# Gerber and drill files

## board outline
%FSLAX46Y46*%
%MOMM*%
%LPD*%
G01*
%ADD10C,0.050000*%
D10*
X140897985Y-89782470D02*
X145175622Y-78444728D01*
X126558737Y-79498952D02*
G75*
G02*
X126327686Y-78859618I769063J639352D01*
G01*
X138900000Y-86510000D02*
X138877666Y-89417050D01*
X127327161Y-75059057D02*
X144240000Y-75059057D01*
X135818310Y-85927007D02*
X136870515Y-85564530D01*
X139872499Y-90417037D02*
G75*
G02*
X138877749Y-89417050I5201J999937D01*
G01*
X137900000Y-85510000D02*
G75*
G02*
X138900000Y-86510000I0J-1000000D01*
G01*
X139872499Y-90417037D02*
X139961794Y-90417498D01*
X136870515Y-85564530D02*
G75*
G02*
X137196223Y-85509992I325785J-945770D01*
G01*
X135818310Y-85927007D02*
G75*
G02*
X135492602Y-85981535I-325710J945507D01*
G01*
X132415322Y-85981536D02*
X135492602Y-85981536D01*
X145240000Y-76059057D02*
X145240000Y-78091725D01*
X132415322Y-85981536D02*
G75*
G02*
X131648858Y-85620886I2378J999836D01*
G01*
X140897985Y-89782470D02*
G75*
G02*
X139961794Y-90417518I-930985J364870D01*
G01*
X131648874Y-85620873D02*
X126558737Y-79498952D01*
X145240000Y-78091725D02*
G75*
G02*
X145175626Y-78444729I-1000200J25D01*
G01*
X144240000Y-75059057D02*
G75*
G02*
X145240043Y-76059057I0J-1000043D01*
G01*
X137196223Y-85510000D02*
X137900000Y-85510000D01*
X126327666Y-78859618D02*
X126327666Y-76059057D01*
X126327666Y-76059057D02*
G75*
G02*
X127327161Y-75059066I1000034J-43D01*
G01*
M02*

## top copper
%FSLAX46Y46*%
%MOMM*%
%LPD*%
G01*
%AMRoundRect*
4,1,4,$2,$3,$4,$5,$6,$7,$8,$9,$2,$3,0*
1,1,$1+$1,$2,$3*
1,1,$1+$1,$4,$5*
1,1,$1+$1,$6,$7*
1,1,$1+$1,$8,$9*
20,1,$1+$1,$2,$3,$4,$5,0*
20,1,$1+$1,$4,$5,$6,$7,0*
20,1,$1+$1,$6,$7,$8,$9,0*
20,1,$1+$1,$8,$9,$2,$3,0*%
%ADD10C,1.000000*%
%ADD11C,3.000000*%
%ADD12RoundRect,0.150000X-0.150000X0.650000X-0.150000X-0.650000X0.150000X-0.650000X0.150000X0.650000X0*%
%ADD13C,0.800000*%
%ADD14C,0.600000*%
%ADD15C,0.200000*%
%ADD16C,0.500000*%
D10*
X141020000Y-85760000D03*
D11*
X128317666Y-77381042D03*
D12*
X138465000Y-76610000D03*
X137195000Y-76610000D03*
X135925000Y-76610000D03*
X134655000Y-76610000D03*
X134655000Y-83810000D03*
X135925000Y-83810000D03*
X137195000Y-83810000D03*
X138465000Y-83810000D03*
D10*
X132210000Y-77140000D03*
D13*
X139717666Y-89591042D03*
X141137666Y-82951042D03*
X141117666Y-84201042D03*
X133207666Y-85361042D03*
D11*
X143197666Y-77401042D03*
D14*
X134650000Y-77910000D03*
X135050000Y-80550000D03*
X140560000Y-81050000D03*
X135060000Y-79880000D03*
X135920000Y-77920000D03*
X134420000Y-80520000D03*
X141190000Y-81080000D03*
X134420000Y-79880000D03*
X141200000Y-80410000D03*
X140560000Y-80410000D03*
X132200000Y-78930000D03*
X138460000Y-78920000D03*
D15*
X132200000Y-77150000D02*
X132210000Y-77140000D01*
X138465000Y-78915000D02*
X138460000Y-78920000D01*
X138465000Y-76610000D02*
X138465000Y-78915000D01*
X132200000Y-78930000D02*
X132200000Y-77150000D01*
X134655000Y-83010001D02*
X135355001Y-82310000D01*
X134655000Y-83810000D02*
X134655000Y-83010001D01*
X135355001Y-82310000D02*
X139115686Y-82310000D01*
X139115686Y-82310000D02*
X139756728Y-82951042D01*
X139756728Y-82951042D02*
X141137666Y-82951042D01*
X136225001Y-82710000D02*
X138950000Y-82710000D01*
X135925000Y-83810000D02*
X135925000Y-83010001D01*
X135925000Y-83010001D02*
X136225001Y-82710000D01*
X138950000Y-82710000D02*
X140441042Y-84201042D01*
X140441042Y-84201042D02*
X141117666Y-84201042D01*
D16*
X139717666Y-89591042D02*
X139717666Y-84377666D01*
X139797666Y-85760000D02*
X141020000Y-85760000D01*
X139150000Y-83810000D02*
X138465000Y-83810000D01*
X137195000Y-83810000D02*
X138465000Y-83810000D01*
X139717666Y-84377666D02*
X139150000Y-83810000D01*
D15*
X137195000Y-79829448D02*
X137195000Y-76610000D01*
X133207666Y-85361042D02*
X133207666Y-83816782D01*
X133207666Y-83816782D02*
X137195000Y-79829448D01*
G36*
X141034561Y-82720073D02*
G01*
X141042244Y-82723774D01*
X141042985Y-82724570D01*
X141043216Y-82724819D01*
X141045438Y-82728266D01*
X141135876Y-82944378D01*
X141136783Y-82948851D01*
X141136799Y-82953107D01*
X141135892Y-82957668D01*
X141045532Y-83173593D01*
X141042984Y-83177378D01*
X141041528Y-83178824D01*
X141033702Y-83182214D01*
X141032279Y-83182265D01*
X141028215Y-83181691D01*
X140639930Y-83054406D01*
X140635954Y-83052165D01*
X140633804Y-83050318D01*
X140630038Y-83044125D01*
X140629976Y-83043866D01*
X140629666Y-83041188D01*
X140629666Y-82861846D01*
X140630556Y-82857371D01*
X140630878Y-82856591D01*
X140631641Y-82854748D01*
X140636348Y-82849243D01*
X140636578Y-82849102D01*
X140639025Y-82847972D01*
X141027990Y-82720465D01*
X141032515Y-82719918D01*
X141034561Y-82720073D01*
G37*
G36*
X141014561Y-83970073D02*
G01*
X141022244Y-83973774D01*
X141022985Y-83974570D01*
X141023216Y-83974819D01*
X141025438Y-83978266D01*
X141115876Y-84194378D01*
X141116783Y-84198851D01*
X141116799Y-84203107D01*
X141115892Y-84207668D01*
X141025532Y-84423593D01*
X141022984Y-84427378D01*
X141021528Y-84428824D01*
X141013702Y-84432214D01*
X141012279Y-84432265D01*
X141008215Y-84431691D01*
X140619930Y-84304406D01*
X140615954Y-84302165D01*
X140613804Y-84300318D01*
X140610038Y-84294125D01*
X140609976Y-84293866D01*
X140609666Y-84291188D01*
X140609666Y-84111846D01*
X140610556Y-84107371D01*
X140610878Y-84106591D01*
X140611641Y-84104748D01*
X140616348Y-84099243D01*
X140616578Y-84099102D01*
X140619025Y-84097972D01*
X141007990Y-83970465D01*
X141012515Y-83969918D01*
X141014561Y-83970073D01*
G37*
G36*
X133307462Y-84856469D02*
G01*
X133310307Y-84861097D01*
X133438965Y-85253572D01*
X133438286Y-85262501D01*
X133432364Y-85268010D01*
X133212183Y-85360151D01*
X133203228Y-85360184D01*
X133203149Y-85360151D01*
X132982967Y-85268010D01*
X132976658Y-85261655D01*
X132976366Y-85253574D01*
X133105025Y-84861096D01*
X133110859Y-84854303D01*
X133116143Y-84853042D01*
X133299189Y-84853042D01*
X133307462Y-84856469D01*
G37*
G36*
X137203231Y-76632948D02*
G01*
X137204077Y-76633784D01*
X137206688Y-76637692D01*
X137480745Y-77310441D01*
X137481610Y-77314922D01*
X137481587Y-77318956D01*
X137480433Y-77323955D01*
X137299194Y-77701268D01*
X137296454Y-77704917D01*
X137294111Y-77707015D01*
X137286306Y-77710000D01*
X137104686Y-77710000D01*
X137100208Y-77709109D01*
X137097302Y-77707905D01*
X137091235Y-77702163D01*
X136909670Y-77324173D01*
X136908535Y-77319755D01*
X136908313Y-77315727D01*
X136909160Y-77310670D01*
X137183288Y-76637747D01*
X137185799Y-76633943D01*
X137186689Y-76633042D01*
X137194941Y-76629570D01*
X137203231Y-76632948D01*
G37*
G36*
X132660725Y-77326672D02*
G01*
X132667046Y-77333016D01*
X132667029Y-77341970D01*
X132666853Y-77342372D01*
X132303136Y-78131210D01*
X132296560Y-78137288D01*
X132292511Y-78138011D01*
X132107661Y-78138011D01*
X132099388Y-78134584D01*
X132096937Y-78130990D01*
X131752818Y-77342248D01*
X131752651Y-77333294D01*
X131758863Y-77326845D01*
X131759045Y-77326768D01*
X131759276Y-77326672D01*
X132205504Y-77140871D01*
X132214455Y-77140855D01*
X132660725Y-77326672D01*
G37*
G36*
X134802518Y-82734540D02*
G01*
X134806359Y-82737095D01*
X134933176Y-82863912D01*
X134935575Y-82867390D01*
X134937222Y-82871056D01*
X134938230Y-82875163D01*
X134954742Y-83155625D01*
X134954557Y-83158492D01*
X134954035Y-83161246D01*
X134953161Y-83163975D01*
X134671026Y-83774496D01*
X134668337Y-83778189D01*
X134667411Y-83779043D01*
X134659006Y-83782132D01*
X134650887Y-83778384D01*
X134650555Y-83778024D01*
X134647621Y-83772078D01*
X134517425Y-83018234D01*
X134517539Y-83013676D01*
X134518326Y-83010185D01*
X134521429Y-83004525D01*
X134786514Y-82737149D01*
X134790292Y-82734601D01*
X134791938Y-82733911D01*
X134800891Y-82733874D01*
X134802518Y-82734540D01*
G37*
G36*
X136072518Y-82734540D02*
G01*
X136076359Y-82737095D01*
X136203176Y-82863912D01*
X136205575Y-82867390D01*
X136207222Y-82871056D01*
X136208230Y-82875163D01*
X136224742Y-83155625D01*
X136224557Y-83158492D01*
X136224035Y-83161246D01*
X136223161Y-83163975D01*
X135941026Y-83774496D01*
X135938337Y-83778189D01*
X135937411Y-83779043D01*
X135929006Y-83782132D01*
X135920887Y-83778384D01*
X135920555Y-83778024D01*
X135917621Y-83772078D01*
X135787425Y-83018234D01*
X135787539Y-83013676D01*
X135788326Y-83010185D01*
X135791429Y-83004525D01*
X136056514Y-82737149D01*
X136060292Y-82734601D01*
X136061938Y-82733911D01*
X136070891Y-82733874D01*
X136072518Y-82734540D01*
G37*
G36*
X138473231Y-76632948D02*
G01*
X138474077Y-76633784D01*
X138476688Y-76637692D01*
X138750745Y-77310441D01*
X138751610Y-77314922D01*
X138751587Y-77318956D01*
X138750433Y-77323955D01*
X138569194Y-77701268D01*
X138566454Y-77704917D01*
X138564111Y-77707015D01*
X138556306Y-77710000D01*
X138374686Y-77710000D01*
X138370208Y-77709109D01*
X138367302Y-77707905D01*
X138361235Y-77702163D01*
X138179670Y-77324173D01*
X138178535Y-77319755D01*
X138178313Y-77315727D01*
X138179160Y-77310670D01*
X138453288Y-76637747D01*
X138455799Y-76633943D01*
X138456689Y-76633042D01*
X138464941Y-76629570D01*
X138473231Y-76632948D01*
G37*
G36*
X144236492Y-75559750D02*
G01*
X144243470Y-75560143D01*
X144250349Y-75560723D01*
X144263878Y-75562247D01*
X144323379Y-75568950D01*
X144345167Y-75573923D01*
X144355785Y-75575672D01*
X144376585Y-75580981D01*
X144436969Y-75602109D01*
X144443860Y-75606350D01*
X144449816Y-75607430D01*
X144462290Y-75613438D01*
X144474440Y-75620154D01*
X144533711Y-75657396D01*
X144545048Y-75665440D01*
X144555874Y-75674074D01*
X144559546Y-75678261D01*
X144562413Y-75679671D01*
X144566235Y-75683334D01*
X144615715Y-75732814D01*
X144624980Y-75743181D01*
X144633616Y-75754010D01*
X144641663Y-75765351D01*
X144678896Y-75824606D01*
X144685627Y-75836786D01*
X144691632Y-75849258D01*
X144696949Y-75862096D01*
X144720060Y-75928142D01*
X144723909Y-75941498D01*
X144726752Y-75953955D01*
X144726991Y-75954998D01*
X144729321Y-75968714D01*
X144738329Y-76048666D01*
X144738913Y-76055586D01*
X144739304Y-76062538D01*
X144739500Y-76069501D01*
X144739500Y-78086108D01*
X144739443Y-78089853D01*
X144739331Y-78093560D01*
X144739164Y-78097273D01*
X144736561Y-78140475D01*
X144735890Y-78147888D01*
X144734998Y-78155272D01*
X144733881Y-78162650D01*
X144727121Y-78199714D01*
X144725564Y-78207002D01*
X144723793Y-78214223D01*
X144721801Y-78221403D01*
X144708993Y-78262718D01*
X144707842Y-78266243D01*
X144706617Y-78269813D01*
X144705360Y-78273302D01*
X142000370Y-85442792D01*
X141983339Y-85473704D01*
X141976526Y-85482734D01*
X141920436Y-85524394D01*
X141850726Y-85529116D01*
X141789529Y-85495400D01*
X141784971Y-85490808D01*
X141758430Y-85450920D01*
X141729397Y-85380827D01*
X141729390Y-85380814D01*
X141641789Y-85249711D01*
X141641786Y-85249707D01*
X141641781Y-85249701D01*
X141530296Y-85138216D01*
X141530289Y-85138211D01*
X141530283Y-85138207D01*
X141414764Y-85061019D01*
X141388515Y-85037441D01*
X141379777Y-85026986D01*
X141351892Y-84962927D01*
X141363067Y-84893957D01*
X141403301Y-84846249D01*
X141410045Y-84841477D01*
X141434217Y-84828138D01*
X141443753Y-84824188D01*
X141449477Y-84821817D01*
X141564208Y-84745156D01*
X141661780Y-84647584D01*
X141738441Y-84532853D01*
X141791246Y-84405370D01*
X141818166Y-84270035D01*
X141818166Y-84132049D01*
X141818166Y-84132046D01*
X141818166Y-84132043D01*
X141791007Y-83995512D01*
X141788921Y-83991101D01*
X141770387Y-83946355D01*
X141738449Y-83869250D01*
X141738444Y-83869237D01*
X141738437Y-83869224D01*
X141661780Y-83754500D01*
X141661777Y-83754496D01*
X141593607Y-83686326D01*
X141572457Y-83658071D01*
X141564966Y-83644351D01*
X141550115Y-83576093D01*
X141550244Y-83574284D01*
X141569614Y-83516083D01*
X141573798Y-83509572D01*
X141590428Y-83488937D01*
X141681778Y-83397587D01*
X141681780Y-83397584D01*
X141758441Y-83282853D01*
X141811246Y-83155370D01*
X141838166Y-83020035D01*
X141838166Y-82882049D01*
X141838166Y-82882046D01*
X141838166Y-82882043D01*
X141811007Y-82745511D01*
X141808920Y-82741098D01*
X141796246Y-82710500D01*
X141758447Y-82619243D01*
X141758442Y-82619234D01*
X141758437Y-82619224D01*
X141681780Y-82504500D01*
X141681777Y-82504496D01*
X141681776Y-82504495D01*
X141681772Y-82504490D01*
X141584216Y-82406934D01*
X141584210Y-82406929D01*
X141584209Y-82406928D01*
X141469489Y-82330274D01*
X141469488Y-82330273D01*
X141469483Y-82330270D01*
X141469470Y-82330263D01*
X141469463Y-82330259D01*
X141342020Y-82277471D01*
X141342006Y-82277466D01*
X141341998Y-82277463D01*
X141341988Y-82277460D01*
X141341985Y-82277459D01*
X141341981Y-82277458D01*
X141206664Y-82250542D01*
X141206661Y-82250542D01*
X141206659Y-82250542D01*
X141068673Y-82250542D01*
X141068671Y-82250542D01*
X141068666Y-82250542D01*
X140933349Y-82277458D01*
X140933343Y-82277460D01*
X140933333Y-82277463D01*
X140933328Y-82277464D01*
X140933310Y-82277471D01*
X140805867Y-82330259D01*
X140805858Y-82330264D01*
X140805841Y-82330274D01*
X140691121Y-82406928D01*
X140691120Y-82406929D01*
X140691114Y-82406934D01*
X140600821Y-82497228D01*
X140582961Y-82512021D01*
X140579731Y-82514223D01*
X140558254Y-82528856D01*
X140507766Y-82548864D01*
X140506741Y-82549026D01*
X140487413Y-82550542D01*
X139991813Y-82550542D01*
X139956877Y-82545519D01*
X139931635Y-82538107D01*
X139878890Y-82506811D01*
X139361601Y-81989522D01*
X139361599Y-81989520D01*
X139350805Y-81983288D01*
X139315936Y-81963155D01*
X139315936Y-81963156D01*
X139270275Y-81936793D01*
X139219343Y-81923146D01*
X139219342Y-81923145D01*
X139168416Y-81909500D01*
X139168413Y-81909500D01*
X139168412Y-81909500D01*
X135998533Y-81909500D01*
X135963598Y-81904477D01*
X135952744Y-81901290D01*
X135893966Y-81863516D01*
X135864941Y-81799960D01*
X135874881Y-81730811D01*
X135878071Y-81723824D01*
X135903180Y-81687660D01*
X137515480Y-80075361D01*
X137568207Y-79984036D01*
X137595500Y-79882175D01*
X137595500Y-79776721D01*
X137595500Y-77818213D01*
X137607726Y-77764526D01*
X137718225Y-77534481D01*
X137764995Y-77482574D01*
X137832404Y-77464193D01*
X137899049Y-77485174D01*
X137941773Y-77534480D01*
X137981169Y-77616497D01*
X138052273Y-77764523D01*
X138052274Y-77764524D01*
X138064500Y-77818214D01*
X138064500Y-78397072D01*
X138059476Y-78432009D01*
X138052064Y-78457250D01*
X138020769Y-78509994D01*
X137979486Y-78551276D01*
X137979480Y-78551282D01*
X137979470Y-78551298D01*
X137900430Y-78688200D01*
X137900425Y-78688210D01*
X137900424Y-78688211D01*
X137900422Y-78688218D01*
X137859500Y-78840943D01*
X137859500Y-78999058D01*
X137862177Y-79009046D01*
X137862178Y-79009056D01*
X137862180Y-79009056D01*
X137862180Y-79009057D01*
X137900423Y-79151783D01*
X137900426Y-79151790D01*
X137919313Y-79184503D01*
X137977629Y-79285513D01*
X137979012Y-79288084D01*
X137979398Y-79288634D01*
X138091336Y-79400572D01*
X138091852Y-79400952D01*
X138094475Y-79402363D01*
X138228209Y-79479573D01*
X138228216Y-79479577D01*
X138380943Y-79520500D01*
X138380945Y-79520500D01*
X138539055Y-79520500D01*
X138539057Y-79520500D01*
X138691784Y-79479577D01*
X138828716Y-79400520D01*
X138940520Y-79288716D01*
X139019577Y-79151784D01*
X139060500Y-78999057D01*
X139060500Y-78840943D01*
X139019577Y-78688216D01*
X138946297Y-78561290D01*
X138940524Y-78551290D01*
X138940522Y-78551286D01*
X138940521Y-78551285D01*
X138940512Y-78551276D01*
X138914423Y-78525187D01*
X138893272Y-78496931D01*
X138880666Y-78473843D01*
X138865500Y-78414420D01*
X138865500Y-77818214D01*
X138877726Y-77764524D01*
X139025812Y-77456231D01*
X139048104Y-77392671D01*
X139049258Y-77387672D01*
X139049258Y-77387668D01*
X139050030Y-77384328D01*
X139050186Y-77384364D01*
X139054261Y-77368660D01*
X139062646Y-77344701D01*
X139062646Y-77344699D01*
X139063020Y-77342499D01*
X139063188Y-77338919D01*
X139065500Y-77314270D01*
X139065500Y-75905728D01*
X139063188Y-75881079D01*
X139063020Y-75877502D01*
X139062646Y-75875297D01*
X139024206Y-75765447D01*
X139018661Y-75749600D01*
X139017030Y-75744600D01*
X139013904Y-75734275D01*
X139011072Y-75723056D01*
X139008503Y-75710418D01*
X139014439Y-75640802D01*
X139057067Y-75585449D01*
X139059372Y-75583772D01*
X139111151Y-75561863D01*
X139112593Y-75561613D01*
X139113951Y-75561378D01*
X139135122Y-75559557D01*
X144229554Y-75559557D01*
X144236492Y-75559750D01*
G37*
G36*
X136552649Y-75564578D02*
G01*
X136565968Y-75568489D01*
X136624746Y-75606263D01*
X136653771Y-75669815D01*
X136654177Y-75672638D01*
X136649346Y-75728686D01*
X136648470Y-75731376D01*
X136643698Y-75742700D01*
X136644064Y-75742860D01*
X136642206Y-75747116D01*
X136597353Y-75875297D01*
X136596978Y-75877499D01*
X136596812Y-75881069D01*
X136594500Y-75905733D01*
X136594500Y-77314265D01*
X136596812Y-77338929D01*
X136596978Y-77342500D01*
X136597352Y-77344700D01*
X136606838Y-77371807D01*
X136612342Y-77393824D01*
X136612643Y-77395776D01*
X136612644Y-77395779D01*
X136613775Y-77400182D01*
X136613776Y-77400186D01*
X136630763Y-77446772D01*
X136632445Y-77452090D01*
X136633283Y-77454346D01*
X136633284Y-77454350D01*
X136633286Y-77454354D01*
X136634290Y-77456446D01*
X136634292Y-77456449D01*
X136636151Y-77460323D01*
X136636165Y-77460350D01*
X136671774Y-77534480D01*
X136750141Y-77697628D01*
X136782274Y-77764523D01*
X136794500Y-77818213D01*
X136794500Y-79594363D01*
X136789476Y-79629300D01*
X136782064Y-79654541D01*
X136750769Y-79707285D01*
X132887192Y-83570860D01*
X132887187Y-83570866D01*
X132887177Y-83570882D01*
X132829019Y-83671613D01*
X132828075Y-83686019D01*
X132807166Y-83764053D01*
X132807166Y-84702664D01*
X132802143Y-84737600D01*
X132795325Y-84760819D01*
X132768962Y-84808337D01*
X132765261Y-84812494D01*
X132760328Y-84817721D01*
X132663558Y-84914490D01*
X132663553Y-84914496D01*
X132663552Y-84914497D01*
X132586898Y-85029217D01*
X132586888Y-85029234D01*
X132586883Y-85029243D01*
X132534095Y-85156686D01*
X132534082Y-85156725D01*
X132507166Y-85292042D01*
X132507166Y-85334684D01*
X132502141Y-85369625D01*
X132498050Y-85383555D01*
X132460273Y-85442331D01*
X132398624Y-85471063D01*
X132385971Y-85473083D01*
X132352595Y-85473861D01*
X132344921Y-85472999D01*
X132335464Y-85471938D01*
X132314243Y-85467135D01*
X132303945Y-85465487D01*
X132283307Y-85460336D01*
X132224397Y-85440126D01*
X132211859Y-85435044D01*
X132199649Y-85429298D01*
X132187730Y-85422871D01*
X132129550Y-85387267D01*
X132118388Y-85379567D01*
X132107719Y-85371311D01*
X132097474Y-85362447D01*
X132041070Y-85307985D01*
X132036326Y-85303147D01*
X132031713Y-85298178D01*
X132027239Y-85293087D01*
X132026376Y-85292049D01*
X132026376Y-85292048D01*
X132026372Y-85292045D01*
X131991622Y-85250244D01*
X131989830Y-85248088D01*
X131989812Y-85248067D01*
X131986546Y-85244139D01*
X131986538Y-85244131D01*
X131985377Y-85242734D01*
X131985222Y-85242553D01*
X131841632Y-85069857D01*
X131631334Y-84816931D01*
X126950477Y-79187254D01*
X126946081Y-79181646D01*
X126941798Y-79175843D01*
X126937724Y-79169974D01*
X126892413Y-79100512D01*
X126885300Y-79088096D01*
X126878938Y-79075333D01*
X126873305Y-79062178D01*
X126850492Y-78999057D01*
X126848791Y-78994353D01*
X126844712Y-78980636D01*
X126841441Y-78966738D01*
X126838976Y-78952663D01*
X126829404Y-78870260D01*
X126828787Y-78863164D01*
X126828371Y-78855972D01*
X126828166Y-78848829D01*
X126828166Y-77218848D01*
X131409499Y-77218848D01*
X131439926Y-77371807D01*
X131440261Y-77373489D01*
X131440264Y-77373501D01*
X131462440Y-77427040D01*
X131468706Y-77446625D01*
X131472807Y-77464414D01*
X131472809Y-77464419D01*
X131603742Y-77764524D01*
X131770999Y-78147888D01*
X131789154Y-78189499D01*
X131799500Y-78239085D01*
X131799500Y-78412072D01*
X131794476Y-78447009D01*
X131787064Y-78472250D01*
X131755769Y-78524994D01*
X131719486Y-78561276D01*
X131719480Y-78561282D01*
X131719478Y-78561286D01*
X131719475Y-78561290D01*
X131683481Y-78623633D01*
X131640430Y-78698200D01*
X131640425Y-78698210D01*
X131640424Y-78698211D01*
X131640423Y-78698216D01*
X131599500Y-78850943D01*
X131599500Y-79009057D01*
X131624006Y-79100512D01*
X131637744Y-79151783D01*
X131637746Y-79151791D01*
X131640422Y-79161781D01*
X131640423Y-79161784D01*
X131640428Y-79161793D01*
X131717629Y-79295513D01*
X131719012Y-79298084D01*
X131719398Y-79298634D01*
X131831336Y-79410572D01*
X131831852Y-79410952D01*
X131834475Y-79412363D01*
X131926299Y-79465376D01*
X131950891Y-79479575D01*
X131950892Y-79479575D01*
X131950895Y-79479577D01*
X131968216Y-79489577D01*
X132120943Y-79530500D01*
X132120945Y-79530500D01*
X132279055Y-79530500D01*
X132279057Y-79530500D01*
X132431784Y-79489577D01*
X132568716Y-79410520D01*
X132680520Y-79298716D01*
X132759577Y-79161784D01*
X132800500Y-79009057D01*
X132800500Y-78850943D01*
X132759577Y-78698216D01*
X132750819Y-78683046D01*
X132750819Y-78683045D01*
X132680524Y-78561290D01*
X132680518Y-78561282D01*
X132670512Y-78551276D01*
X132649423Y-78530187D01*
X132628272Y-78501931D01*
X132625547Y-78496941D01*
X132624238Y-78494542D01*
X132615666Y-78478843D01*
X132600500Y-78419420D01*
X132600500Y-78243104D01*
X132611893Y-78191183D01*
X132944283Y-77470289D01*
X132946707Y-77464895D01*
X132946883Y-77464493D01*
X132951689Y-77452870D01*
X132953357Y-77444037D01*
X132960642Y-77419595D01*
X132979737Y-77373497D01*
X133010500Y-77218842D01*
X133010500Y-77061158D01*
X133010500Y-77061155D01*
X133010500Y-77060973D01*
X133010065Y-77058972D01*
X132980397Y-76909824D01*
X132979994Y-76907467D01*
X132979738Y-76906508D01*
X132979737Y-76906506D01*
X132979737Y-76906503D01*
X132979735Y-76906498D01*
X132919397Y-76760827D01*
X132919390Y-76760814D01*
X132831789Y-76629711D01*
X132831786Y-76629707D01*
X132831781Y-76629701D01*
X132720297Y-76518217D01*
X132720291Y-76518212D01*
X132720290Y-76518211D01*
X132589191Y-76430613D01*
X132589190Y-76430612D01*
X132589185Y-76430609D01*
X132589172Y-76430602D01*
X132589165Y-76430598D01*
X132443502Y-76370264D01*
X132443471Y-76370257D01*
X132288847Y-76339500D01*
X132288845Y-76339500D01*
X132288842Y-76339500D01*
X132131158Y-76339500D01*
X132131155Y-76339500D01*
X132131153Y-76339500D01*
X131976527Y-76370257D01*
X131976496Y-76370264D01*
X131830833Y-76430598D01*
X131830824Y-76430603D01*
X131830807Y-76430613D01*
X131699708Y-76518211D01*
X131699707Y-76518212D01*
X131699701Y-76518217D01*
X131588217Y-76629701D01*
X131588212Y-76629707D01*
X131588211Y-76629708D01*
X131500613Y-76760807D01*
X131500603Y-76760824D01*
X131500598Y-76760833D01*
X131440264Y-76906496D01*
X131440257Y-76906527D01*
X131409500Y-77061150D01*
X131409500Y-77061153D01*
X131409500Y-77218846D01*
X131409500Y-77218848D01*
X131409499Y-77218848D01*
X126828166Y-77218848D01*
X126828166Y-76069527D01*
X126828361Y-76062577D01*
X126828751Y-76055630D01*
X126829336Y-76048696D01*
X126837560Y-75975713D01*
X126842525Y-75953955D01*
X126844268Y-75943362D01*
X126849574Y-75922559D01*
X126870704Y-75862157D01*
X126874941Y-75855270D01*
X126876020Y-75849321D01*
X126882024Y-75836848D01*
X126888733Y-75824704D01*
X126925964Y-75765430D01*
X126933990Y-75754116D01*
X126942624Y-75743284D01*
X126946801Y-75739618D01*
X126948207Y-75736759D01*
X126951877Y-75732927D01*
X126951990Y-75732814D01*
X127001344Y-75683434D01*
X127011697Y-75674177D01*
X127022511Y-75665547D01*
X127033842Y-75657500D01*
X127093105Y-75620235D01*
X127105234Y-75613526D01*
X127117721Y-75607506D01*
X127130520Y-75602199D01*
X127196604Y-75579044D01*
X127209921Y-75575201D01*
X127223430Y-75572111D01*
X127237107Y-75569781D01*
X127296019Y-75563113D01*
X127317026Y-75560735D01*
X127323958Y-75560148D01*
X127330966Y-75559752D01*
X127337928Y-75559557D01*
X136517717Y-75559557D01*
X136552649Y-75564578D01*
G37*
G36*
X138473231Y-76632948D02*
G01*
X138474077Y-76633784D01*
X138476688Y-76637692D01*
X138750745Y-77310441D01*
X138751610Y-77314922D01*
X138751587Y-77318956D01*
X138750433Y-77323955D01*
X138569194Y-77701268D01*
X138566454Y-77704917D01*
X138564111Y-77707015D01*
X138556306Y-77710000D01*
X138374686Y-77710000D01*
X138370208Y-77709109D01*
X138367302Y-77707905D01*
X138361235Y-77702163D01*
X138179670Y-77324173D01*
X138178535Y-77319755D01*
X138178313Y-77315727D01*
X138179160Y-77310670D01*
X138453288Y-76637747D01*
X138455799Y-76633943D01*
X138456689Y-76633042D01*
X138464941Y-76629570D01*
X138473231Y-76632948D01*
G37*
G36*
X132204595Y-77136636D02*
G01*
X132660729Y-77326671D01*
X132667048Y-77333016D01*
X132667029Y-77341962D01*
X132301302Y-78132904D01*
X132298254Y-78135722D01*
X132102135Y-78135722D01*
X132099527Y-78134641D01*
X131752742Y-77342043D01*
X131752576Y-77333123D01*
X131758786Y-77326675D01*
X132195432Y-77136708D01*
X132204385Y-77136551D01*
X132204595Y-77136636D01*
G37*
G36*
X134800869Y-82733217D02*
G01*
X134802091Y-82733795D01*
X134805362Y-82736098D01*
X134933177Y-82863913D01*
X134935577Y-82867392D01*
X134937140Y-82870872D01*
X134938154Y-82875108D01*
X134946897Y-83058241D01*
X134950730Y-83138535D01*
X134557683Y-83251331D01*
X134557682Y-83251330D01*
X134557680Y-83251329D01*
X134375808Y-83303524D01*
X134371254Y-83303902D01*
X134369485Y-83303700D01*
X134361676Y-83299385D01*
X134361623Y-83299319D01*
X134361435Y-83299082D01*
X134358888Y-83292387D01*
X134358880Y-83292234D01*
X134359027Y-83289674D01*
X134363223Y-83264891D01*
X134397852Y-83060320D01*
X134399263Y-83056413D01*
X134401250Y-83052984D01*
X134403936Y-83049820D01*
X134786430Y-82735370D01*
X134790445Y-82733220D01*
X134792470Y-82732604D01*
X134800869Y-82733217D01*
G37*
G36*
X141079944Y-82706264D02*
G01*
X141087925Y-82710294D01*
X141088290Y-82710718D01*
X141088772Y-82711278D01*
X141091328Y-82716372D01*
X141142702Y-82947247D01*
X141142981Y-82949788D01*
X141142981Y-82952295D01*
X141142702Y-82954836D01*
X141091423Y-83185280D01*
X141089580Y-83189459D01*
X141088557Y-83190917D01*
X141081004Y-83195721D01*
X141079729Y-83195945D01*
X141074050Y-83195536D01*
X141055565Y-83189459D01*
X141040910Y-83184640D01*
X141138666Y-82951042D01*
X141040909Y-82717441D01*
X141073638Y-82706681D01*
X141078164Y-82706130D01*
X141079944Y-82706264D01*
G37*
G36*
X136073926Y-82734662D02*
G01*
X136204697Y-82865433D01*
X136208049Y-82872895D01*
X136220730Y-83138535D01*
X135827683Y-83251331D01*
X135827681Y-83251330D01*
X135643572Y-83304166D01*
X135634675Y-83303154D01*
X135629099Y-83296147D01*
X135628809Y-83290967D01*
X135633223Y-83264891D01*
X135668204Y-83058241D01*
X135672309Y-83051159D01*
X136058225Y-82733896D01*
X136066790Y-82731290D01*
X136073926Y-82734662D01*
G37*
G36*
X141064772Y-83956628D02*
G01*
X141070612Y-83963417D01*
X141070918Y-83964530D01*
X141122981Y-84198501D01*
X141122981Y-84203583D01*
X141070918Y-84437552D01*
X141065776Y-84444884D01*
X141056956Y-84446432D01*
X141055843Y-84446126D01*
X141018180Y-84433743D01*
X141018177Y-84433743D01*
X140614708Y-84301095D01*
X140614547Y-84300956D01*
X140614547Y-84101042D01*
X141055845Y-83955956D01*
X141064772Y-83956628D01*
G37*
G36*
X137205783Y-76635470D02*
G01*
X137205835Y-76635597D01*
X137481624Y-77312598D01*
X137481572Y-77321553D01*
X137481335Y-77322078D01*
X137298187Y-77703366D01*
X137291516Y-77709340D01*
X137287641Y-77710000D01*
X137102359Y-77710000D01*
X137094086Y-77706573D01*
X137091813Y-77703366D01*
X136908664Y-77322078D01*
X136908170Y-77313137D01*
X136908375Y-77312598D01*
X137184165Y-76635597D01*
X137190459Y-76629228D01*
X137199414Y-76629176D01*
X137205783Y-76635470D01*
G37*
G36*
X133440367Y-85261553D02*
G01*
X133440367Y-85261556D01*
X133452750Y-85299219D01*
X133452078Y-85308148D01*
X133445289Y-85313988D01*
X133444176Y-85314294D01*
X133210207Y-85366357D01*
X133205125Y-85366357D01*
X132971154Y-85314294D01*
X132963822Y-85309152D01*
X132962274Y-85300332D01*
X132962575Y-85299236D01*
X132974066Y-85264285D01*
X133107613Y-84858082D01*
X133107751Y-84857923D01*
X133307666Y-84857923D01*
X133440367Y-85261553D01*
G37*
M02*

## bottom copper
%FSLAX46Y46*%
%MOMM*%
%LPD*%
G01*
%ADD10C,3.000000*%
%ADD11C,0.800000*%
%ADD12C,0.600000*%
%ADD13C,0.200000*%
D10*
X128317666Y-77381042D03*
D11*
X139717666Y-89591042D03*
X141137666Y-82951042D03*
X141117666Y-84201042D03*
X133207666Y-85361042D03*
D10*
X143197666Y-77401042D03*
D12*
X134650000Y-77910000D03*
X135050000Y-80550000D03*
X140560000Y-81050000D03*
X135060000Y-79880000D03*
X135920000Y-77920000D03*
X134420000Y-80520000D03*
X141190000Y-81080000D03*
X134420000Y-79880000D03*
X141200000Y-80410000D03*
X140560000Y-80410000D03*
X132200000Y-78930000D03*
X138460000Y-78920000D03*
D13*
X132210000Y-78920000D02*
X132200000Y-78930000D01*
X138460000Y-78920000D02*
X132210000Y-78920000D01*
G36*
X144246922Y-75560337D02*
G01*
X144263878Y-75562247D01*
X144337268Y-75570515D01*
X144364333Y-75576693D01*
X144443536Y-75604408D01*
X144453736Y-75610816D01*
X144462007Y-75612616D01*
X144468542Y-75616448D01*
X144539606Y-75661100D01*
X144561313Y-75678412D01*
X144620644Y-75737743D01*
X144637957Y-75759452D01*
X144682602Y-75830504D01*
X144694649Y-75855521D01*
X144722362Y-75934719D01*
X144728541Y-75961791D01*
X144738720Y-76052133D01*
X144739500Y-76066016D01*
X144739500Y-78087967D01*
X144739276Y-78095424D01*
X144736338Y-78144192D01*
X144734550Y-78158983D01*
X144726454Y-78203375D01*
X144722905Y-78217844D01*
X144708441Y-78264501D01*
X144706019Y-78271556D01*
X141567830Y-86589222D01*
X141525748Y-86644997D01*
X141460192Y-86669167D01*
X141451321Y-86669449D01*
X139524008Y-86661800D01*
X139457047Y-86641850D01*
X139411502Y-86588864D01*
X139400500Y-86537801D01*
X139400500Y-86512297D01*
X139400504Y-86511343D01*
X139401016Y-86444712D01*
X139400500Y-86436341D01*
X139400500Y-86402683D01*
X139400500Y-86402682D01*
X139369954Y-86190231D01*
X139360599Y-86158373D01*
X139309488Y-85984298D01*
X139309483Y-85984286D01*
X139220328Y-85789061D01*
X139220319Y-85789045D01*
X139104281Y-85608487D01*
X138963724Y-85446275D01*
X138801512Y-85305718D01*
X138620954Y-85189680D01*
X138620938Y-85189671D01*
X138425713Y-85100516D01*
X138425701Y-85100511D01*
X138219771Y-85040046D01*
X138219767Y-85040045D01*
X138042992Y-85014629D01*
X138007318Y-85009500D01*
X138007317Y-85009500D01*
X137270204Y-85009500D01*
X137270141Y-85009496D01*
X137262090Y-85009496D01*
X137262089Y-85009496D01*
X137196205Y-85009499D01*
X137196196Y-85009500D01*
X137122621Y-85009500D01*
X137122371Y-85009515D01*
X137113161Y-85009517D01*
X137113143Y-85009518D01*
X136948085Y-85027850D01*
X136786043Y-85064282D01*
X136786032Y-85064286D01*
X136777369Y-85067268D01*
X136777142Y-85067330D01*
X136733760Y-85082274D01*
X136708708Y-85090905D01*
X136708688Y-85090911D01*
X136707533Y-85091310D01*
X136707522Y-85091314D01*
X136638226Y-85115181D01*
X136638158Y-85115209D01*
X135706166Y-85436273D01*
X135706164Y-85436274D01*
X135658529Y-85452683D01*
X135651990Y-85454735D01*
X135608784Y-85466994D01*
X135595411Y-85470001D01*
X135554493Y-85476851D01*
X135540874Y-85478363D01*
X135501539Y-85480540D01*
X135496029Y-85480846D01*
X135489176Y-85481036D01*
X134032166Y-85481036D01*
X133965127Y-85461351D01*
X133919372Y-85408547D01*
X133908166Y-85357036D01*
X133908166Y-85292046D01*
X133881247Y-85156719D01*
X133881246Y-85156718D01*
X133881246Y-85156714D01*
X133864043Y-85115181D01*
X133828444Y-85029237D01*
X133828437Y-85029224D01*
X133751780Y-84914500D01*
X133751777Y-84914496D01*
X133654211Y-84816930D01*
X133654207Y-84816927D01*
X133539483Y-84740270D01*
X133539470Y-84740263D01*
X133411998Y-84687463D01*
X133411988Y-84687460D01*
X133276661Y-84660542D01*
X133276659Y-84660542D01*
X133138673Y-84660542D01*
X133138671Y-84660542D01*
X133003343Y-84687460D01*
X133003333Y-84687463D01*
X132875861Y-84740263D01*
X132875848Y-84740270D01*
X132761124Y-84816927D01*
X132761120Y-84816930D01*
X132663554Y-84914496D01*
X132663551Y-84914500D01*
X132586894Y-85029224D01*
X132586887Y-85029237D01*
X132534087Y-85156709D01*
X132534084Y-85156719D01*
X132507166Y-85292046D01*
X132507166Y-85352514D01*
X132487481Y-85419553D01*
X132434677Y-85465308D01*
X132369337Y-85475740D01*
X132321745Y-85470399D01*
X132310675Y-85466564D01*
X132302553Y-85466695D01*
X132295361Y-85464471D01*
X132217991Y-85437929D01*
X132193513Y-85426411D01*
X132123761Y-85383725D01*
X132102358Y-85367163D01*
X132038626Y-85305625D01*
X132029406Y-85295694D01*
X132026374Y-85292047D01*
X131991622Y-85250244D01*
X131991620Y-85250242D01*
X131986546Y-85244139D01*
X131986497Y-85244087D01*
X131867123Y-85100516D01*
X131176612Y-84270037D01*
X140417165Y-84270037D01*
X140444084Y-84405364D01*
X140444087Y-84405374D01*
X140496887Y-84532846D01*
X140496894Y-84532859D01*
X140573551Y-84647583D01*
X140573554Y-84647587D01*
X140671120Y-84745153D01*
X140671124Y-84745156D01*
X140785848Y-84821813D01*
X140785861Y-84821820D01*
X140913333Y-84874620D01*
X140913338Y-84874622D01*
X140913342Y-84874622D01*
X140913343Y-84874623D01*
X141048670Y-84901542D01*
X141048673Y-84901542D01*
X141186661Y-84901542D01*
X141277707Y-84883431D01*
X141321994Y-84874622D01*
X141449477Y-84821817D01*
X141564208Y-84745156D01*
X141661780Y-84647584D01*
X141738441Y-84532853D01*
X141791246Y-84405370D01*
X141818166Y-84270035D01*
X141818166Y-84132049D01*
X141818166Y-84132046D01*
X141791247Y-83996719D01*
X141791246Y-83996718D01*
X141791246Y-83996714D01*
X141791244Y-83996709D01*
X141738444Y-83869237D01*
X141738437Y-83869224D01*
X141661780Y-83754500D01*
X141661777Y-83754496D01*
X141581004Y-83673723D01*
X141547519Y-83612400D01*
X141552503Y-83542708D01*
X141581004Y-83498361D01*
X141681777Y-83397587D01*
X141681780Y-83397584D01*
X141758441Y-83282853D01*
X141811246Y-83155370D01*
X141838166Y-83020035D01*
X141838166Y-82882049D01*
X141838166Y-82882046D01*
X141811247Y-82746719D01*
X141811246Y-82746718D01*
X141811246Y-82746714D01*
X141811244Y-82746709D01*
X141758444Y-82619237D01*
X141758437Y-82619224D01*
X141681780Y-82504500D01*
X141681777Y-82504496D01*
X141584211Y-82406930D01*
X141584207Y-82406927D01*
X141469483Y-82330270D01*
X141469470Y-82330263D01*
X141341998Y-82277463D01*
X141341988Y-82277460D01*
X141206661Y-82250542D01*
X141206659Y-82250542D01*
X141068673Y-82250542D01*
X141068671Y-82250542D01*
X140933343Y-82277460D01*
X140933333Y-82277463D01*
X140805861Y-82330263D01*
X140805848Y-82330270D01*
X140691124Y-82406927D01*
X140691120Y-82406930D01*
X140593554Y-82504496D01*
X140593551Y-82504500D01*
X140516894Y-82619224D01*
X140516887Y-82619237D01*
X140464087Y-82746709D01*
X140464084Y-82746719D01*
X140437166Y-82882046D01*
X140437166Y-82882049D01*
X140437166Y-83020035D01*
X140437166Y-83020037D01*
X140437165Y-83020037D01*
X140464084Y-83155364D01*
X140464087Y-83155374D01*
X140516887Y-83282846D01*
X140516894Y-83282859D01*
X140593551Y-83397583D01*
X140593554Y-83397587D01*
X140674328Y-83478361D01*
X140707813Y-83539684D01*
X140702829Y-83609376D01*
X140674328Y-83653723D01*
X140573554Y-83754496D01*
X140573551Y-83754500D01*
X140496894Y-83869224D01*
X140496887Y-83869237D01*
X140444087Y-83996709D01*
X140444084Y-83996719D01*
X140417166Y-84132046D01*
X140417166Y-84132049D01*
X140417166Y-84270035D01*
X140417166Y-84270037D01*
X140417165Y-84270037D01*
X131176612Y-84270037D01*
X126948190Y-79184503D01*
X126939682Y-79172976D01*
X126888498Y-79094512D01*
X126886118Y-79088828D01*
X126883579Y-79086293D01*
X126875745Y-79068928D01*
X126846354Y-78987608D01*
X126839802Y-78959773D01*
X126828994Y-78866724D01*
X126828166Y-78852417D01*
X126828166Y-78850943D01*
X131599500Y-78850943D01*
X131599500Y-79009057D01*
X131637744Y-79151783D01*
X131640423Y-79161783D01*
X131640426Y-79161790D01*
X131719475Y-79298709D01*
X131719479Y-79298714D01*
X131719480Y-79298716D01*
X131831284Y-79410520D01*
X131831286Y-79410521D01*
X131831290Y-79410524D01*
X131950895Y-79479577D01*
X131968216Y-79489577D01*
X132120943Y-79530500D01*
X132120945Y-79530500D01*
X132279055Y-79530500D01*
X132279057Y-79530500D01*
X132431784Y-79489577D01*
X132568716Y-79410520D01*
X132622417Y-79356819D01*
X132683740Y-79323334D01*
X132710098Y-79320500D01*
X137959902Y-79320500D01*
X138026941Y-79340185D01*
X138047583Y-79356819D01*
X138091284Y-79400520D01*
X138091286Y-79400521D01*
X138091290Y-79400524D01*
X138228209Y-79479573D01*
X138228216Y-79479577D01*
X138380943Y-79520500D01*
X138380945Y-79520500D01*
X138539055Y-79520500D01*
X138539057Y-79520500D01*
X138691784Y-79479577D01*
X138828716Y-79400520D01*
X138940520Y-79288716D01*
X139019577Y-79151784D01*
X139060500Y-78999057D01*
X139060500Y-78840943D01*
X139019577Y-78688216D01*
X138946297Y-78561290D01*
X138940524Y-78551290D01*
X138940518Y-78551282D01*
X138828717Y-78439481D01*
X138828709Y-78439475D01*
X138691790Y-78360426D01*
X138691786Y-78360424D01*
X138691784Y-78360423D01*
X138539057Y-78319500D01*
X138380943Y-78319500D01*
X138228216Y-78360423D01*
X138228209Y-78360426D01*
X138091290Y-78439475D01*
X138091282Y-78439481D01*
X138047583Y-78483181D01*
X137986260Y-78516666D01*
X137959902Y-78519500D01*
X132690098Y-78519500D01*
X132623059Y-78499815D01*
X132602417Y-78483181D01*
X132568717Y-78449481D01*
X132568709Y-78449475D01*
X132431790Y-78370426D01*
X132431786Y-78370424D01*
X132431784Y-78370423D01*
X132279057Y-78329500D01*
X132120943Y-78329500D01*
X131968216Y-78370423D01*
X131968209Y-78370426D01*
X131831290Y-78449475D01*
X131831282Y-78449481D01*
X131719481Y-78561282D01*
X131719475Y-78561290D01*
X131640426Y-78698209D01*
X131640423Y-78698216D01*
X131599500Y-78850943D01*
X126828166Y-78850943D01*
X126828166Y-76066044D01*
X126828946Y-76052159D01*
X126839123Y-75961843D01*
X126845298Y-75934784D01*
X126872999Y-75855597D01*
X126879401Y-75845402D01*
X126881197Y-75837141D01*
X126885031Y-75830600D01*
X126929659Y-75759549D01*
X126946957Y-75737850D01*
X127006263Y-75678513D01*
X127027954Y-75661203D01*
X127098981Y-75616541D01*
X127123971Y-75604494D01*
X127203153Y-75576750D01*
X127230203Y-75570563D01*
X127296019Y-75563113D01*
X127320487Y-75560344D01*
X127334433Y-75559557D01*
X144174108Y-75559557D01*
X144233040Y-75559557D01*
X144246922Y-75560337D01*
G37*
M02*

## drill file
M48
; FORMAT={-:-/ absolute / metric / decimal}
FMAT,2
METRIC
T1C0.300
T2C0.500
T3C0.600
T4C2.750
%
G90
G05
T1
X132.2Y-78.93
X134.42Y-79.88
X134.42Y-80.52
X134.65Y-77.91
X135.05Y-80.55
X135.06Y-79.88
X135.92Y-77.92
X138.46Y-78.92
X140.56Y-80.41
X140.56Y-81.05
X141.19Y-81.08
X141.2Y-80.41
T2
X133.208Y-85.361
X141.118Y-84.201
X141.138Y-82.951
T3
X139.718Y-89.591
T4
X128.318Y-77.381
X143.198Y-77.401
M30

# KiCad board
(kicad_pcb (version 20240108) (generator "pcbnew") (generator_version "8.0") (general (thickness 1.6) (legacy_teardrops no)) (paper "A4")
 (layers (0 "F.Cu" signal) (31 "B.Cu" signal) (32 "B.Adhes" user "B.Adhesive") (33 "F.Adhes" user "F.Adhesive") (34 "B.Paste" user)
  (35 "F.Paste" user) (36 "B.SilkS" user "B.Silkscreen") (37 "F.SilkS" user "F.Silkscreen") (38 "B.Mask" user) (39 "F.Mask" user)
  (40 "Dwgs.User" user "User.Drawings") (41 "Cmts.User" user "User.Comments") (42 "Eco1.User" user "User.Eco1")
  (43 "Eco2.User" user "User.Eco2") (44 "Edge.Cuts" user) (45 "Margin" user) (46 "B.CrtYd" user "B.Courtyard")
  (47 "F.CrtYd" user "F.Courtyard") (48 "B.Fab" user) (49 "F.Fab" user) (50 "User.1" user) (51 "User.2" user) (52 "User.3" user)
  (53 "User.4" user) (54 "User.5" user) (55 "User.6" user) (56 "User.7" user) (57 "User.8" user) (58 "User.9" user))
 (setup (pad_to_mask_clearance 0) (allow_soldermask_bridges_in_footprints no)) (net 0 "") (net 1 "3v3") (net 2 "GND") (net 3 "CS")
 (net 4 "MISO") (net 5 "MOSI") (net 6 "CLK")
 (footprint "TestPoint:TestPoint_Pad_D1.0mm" (layer "F.Cu") (at 141.02 85.76)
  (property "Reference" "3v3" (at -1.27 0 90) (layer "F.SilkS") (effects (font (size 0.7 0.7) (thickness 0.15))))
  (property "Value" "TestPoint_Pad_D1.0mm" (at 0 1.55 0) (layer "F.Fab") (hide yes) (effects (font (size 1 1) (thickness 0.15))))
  (pad "1" smd circle (at 0 0) (size 1 1) (layers "F.Cu" "F.Mask") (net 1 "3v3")))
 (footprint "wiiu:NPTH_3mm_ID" (layer "F.Cu") (at 128.317666 77.381042)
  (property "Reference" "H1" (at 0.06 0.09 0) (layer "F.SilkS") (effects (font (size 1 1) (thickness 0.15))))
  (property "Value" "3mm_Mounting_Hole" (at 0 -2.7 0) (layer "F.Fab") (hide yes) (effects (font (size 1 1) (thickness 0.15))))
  (pad "" thru_hole circle (at 0 0) (size 3 3) (drill 2.75) (layers "*.Cu" "*.Mask") (remove_unused_layers no) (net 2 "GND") (clearance 1.6)
   (zone_connect 2)))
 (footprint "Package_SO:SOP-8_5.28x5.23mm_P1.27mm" (layer "F.Cu") (at 136.56 80.21 -90)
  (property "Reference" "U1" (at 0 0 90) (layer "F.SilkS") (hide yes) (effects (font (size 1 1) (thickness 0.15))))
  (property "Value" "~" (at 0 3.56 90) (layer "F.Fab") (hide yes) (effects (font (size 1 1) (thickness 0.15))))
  (pad "1" smd roundrect (at -3.6 -1.905 270) (size 1.6 0.6) (layers "F.Cu" "F.Paste" "F.Mask") (roundrect_rratio 0.25) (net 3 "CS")
   (teardrops (best_length_ratio 0.5) (max_length 1) (best_width_ratio 1) (max_width 2) (curve_points 0) (filter_ratio 0.9) (enabled yes)
    (allow_two_segments yes) (prefer_zone_connections yes)))
  (pad "2" smd roundrect (at -3.6 -0.635 270) (size 1.6 0.6) (layers "F.Cu" "F.Paste" "F.Mask") (roundrect_rratio 0.25) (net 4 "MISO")
   (teardrops (best_length_ratio 0.5) (max_length 1) (best_width_ratio 1) (max_width 2) (curve_points 0) (filter_ratio 0.9) (enabled yes)
    (allow_two_segments yes) (prefer_zone_connections yes)))
  (pad "3" smd roundrect (at -3.6 0.635 270) (size 1.6 0.6) (layers "F.Cu" "F.Paste" "F.Mask") (roundrect_rratio 0.25) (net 2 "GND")
   (zone_connect 2))
  (pad "4" smd roundrect (at -3.6 1.905 270) (size 1.6 0.6) (layers "F.Cu" "F.Paste" "F.Mask") (roundrect_rratio 0.25) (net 2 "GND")
   (zone_connect 2))
  (pad "5" smd roundrect (at 3.6 1.905 270) (size 1.6 0.6) (layers "F.Cu" "F.Paste" "F.Mask") (roundrect_rratio 0.25) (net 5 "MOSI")
   (teardrops (best_length_ratio 0.5) (max_length 1) (best_width_ratio 1) (max_width 2) (curve_points 0) (filter_ratio 0.9) (enabled yes)
    (allow_two_segments yes) (prefer_zone_connections yes)))
  (pad "6" smd roundrect (at 3.6 0.635 270) (size 1.6 0.6) (layers "F.Cu" "F.Paste" "F.Mask") (roundrect_rratio 0.25) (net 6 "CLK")
   (teardrops (best_length_ratio 0.5) (max_length 1) (best_width_ratio 1) (max_width 2) (curve_points 0) (filter_ratio 0.9) (enabled yes)
    (allow_two_segments yes) (prefer_zone_connections yes)))
  (pad "7" smd roundrect (at 3.6 -0.635 270) (size 1.6 0.6) (layers "F.Cu" "F.Paste" "F.Mask") (roundrect_rratio 0.25) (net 1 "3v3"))
  (pad "8" smd roundrect (at 3.6 -1.905 270) (size 1.6 0.6) (layers "F.Cu" "F.Paste" "F.Mask") (roundrect_rratio 0.25) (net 1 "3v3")))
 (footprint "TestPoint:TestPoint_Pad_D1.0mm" (layer "F.Cu") (at 132.21 77.14)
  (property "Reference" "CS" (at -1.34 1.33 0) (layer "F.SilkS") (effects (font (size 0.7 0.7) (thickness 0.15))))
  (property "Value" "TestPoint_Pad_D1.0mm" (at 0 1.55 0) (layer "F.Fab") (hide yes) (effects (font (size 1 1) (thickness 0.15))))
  (pad "1" smd circle (at 0 0) (size 1 1) (layers "F.Cu" "F.Mask") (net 3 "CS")
   (teardrops (best_length_ratio 0.5) (max_length 1) (best_width_ratio 1) (max_width 2) (curve_points 0) (filter_ratio 0.9) (enabled yes)
    (allow_two_segments yes) (prefer_zone_connections yes))))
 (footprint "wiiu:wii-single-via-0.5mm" (layer "F.Cu") (at 139.717666 89.591042)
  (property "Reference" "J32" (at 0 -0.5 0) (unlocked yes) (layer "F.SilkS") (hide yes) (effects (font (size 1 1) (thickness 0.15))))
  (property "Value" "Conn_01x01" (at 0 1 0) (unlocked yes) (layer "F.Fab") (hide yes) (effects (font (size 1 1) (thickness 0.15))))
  (pad "1" thru_hole circle (at 0 0 270) (size 0.8 0.508) (drill 0.6) (layers "*.Cu" "*.Mask") (remove_unused_layers no) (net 1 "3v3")
   (zone_connect 2)))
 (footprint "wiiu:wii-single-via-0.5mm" (layer "F.Cu") (at 141.137666 82.951042)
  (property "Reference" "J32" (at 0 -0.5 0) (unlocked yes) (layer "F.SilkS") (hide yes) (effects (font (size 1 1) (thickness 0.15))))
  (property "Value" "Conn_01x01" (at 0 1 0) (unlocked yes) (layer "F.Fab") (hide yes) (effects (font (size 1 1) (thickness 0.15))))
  (pad "1" thru_hole circle (at 0 0 270) (size 0.8 0.508) (drill 0.5) (layers "*.Cu" "*.Mask") (remove_unused_layers no) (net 5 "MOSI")
   (teardrops (best_length_ratio 0.5) (max_length 1) (best_width_ratio 1) (max_width 2) (curve_points 0) (filter_ratio 0.9) (enabled yes)
    (allow_two_segments yes) (prefer_zone_connections yes))))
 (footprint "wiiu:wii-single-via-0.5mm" (layer "F.Cu") (at 141.117666 84.201042)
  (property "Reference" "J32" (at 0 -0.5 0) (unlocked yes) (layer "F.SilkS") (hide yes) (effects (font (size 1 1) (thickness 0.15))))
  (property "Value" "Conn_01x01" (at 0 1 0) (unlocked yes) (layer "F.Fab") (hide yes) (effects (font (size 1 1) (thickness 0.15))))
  (pad "1" thru_hole circle (at 0 0 270) (size 0.8 0.508) (drill 0.5) (layers "*.Cu" "*.Mask") (remove_unused_layers no) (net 6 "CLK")
   (teardrops (best_length_ratio 0.5) (max_length 1) (best_width_ratio 1) (max_width 2) (curve_points 0) (filter_ratio 0.9) (enabled yes)
    (allow_two_segments yes) (prefer_zone_connections yes))))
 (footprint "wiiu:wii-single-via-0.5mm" (layer "F.Cu") (at 133.207666 85.361042)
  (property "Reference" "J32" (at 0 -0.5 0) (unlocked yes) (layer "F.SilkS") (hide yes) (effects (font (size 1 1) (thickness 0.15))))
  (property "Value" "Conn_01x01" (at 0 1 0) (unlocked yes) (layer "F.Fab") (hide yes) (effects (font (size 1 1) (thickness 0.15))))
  (pad "1" thru_hole circle (at 0 0 270) (size 0.8 0.508) (drill 0.5) (layers "*.Cu" "*.Mask") (remove_unused_layers no) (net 4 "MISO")
   (teardrops (best_length_ratio 0.5) (max_length 1) (best_width_ratio 1) (max_width 2) (curve_points 0) (filter_ratio 0.9) (enabled yes)
    (allow_two_segments yes) (prefer_zone_connections yes))))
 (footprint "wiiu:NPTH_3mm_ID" (layer "F.Cu") (at 143.197666 77.401042)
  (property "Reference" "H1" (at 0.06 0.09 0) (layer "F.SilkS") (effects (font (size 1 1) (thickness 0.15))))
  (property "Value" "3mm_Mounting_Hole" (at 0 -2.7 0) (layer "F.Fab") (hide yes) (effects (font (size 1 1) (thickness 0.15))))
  (pad "" thru_hole circle (at 0 0) (size 3 3) (drill 2.75) (layers "*.Cu" "*.Mask") (remove_unused_layers no) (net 2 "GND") (clearance 1.6)
   (zone_connect 2)))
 (gr_line (start 140.897985 89.78247) (end 145.175622 78.444728) (stroke (width 0.05) (type default)) (layer "Edge.Cuts"))
 (gr_arc (start 126.558737 79.498952) (mid 126.387214 79.199522) (end 126.327666 78.859618) (stroke (width 0.05) (type default))
  (layer "Edge.Cuts"))
 (gr_line (start 138.9 86.51) (end 138.877666 89.41705) (stroke (width 0.05) (type default)) (layer "Edge.Cuts"))
 (gr_line (start 127.327161 75.059057) (end 144.24 75.059057) (stroke (width 0.05) (type default)) (layer "Edge.Cuts"))
 (gr_line (start 135.81831 85.927007) (end 136.870515 85.56453) (stroke (width 0.05) (type default)) (layer "Edge.Cuts"))
 (gr_arc (start 139.872499 90.417037) (mid 139.168732 90.122328) (end 138.877666 89.41705) (stroke (width 0.05) (type default))
  (layer "Edge.Cuts"))
 (gr_arc (start 137.9 85.51) (mid 138.607107 85.802893) (end 138.9 86.51) (stroke (width 0.05) (type default)) (layer "Edge.Cuts"))
 (gr_line (start 139.872499 90.417037) (end 139.961794 90.417498) (stroke (width 0.05) (type default)) (layer "Edge.Cuts"))
 (gr_arc (start 136.870515 85.56453) (mid 137.031103 85.523731) (end 137.196223 85.51) (stroke (width 0.05) (type default))
  (layer "Edge.Cuts"))
 (gr_arc (start 135.81831 85.927007) (mid 135.657722 85.967809) (end 135.492602 85.981536) (stroke (width 0.05) (type default))
  (layer "Edge.Cuts"))
 (gr_line (start 132.415322 85.981536) (end 135.492602 85.981536) (stroke (width 0.05) (type default)) (layer "Edge.Cuts"))
 (gr_line (start 145.24 76.059057) (end 145.24 78.091725) (stroke (width 0.05) (type default)) (layer "Edge.Cuts"))
 (gr_arc (start 132.415322 85.981536) (mid 131.992015 85.886379) (end 131.648874 85.620873) (stroke (width 0.05) (type default))
  (layer "Edge.Cuts"))
 (gr_arc (start 140.897985 89.78247) (mid 140.52832 90.245099) (end 139.961794 90.417498) (stroke (width 0.05) (type default))
  (layer "Edge.Cuts"))
 (gr_line (start 131.648874 85.620873) (end 126.558737 79.498952) (stroke (width 0.05) (type default)) (layer "Edge.Cuts"))
 (gr_arc (start 145.24 78.091725) (mid 145.22377 78.271137) (end 145.175622 78.444728) (stroke (width 0.05) (type default))
  (layer "Edge.Cuts"))
 (gr_arc (start 144.24 75.059057) (mid 144.947107 75.35195) (end 145.24 76.059057) (stroke (width 0.05) (type default)) (layer "Edge.Cuts"))
 (gr_line (start 137.196223 85.51) (end 137.9 85.51) (stroke (width 0.05) (type default)) (layer "Edge.Cuts"))
 (gr_line (start 126.327666 78.859618) (end 126.327666 76.059057) (stroke (width 0.05) (type default)) (layer "Edge.Cuts"))
 (gr_arc (start 126.327666 76.059057) (mid 126.620394 75.352145) (end 127.327161 75.059057) (stroke (width 0.05) (type default))
  (layer "Edge.Cuts"))
 (via (at 134.65 77.91) (size 0.6) (drill 0.3) (layers "F.Cu" "B.Cu") (free yes) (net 2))
 (via (at 135.05 80.55) (size 0.6) (drill 0.3) (layers "F.Cu" "B.Cu") (free yes) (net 2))
 (via (at 140.56 81.05) (size 0.6) (drill 0.3) (layers "F.Cu" "B.Cu") (free yes) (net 2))
 (via (at 135.06 79.88) (size 0.6) (drill 0.3) (layers "F.Cu" "B.Cu") (free yes) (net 2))
 (via (at 135.92 77.92) (size 0.6) (drill 0.3) (layers "F.Cu" "B.Cu") (free yes) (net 2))
 (via (at 134.42 80.52) (size 0.6) (drill 0.3) (layers "F.Cu" "B.Cu") (free yes) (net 2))
 (via (at 141.19 81.08) (size 0.6) (drill 0.3) (layers "F.Cu" "B.Cu") (free yes) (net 2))
 (via (at 134.42 79.88) (size 0.6) (drill 0.3) (layers "F.Cu" "B.Cu") (free yes) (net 2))
 (via (at 141.2 80.41) (size 0.6) (drill 0.3) (layers "F.Cu" "B.Cu") (free yes) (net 2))
 (via (at 140.56 80.41) (size 0.6) (drill 0.3) (layers "F.Cu" "B.Cu") (free yes) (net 2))
 (segment (start 132.2 77.15) (end 132.21 77.14) (width 0.2) (layer "F.Cu") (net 3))
 (segment (start 138.465 78.915) (end 138.46 78.92) (width 0.2) (layer "F.Cu") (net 3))
 (segment (start 138.465 76.61) (end 138.465 78.915) (width 0.2) (layer "F.Cu") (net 3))
 (segment (start 132.2 78.93) (end 132.2 77.15) (width 0.2) (layer "F.Cu") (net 3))
 (via (at 132.2 78.93) (size 0.6) (drill 0.3) (layers "F.Cu" "B.Cu") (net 3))
 (via (at 138.46 78.92) (size 0.6) (drill 0.3) (layers "F.Cu" "B.Cu") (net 3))
 (segment (start 132.21 78.92) (end 132.2 78.93) (width 0.2) (layer "B.Cu") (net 3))
 (segment (start 138.46 78.92) (end 132.21 78.92) (width 0.2) (layer "B.Cu") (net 3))
 (segment (start 134.655 83.010001) (end 135.355001 82.31) (width 0.2) (layer "F.Cu") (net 5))
 (segment (start 134.655 83.81) (end 134.655 83.010001) (width 0.2) (layer "F.Cu") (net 5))
 (segment (start 135.355001 82.31) (end 139.115686 82.31) (width 0.2) (layer "F.Cu") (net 5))
 (segment (start 139.115686 82.31) (end 139.756728 82.951042) (width 0.2) (layer "F.Cu") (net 5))
 (segment (start 139.756728 82.951042) (end 141.137666 82.951042) (width 0.2) (layer "F.Cu") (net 5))
 (segment (start 136.225001 82.71) (end 138.95 82.71) (width 0.2) (layer "F.Cu") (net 6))
 (segment (start 135.925 83.81) (end 135.925 83.010001) (width 0.2) (layer "F.Cu") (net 6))
 (segment (start 135.925 83.010001) (end 136.225001 82.71) (width 0.2) (layer "F.Cu") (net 6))
 (segment (start 138.95 82.71) (end 140.441042 84.201042) (width 0.2) (layer "F.Cu") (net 6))
 (segment (start 140.441042 84.201042) (end 141.117666 84.201042) (width 0.2) (layer "F.Cu") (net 6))
 (segment (start 139.717666 89.591042) (end 139.717666 84.377666) (width 0.5) (layer "F.Cu") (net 1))
 (segment (start 139.797666 85.76) (end 141.02 85.76) (width 0.5) (layer "F.Cu") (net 1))
 (segment (start 139.15 83.81) (end 138.465 83.81) (width 0.5) (layer "F.Cu") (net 1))
 (segment (start 137.195 83.81) (end 138.465 83.81) (width 0.5) (layer "F.Cu") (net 1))
 (segment (start 139.717666 84.377666) (end 139.15 83.81) (width 0.5) (layer "F.Cu") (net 1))
 (segment (start 137.195 79.829448) (end 137.195 76.61) (width 0.2) (layer "F.Cu") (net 4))
 (segment (start 133.207666 85.361042) (end 133.207666 83.816782) (width 0.2) (layer "F.Cu") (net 4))
 (segment (start 133.207666 83.816782) (end 137.195 79.829448) (width 0.2) (layer "F.Cu") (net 4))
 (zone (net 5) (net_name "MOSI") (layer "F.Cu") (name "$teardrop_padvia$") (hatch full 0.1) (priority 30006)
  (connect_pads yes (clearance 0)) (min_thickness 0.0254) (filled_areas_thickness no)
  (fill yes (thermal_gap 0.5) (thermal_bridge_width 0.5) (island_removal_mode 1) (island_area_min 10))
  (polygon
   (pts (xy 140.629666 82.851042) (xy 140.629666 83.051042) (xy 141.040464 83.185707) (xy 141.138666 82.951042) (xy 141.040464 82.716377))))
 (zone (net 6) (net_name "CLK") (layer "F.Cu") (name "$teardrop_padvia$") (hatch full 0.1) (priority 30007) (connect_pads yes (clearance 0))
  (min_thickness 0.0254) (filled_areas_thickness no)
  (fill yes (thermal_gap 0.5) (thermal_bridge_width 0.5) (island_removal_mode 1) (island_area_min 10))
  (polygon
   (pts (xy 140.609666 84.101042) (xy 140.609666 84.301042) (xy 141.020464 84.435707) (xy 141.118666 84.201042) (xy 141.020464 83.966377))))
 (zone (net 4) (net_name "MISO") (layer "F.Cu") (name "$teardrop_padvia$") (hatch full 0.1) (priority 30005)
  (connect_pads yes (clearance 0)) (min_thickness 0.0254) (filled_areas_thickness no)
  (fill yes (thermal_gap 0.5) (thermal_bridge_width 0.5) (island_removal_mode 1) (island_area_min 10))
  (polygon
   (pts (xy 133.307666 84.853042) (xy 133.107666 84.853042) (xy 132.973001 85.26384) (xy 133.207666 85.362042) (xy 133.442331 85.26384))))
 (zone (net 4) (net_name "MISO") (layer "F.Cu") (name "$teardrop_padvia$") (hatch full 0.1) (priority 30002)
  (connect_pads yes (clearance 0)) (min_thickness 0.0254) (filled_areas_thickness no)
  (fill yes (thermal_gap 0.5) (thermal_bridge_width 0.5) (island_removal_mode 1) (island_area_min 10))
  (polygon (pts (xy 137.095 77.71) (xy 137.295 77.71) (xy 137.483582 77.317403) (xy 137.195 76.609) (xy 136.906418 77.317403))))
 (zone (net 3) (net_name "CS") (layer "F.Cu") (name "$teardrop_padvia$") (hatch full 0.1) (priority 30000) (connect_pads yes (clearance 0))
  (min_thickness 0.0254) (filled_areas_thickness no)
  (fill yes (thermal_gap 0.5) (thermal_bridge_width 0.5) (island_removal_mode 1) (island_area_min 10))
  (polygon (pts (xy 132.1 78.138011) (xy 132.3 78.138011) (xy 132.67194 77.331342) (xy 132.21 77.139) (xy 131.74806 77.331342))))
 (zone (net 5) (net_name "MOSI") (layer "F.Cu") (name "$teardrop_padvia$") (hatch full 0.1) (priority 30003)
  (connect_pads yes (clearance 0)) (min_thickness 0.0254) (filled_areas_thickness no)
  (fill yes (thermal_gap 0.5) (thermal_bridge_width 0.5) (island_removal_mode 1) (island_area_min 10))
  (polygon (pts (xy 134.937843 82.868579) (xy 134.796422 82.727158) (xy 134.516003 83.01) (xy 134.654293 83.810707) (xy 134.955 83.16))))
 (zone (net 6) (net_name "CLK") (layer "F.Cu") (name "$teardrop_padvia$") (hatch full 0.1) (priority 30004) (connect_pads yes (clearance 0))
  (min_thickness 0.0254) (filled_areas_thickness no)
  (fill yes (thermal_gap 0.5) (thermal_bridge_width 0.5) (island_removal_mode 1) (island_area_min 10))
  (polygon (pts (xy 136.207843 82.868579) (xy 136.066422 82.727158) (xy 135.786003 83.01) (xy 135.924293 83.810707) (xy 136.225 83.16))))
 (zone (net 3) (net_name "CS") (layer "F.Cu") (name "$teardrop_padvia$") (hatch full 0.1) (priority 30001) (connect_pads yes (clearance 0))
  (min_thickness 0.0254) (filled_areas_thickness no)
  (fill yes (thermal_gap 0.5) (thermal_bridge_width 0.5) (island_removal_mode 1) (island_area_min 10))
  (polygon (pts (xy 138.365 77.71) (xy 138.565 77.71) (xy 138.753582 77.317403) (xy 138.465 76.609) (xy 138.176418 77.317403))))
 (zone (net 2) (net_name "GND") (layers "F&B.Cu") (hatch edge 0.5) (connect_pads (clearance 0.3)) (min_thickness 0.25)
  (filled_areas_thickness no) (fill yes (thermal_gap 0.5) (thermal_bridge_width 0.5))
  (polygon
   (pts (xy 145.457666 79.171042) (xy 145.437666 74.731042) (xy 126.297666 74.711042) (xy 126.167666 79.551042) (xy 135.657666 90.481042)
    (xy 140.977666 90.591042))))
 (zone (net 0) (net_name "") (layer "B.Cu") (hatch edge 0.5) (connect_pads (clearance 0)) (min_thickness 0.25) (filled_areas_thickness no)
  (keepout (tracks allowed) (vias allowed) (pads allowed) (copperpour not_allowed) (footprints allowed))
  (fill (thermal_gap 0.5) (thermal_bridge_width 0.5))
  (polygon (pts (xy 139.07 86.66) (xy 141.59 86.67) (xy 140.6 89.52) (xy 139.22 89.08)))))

